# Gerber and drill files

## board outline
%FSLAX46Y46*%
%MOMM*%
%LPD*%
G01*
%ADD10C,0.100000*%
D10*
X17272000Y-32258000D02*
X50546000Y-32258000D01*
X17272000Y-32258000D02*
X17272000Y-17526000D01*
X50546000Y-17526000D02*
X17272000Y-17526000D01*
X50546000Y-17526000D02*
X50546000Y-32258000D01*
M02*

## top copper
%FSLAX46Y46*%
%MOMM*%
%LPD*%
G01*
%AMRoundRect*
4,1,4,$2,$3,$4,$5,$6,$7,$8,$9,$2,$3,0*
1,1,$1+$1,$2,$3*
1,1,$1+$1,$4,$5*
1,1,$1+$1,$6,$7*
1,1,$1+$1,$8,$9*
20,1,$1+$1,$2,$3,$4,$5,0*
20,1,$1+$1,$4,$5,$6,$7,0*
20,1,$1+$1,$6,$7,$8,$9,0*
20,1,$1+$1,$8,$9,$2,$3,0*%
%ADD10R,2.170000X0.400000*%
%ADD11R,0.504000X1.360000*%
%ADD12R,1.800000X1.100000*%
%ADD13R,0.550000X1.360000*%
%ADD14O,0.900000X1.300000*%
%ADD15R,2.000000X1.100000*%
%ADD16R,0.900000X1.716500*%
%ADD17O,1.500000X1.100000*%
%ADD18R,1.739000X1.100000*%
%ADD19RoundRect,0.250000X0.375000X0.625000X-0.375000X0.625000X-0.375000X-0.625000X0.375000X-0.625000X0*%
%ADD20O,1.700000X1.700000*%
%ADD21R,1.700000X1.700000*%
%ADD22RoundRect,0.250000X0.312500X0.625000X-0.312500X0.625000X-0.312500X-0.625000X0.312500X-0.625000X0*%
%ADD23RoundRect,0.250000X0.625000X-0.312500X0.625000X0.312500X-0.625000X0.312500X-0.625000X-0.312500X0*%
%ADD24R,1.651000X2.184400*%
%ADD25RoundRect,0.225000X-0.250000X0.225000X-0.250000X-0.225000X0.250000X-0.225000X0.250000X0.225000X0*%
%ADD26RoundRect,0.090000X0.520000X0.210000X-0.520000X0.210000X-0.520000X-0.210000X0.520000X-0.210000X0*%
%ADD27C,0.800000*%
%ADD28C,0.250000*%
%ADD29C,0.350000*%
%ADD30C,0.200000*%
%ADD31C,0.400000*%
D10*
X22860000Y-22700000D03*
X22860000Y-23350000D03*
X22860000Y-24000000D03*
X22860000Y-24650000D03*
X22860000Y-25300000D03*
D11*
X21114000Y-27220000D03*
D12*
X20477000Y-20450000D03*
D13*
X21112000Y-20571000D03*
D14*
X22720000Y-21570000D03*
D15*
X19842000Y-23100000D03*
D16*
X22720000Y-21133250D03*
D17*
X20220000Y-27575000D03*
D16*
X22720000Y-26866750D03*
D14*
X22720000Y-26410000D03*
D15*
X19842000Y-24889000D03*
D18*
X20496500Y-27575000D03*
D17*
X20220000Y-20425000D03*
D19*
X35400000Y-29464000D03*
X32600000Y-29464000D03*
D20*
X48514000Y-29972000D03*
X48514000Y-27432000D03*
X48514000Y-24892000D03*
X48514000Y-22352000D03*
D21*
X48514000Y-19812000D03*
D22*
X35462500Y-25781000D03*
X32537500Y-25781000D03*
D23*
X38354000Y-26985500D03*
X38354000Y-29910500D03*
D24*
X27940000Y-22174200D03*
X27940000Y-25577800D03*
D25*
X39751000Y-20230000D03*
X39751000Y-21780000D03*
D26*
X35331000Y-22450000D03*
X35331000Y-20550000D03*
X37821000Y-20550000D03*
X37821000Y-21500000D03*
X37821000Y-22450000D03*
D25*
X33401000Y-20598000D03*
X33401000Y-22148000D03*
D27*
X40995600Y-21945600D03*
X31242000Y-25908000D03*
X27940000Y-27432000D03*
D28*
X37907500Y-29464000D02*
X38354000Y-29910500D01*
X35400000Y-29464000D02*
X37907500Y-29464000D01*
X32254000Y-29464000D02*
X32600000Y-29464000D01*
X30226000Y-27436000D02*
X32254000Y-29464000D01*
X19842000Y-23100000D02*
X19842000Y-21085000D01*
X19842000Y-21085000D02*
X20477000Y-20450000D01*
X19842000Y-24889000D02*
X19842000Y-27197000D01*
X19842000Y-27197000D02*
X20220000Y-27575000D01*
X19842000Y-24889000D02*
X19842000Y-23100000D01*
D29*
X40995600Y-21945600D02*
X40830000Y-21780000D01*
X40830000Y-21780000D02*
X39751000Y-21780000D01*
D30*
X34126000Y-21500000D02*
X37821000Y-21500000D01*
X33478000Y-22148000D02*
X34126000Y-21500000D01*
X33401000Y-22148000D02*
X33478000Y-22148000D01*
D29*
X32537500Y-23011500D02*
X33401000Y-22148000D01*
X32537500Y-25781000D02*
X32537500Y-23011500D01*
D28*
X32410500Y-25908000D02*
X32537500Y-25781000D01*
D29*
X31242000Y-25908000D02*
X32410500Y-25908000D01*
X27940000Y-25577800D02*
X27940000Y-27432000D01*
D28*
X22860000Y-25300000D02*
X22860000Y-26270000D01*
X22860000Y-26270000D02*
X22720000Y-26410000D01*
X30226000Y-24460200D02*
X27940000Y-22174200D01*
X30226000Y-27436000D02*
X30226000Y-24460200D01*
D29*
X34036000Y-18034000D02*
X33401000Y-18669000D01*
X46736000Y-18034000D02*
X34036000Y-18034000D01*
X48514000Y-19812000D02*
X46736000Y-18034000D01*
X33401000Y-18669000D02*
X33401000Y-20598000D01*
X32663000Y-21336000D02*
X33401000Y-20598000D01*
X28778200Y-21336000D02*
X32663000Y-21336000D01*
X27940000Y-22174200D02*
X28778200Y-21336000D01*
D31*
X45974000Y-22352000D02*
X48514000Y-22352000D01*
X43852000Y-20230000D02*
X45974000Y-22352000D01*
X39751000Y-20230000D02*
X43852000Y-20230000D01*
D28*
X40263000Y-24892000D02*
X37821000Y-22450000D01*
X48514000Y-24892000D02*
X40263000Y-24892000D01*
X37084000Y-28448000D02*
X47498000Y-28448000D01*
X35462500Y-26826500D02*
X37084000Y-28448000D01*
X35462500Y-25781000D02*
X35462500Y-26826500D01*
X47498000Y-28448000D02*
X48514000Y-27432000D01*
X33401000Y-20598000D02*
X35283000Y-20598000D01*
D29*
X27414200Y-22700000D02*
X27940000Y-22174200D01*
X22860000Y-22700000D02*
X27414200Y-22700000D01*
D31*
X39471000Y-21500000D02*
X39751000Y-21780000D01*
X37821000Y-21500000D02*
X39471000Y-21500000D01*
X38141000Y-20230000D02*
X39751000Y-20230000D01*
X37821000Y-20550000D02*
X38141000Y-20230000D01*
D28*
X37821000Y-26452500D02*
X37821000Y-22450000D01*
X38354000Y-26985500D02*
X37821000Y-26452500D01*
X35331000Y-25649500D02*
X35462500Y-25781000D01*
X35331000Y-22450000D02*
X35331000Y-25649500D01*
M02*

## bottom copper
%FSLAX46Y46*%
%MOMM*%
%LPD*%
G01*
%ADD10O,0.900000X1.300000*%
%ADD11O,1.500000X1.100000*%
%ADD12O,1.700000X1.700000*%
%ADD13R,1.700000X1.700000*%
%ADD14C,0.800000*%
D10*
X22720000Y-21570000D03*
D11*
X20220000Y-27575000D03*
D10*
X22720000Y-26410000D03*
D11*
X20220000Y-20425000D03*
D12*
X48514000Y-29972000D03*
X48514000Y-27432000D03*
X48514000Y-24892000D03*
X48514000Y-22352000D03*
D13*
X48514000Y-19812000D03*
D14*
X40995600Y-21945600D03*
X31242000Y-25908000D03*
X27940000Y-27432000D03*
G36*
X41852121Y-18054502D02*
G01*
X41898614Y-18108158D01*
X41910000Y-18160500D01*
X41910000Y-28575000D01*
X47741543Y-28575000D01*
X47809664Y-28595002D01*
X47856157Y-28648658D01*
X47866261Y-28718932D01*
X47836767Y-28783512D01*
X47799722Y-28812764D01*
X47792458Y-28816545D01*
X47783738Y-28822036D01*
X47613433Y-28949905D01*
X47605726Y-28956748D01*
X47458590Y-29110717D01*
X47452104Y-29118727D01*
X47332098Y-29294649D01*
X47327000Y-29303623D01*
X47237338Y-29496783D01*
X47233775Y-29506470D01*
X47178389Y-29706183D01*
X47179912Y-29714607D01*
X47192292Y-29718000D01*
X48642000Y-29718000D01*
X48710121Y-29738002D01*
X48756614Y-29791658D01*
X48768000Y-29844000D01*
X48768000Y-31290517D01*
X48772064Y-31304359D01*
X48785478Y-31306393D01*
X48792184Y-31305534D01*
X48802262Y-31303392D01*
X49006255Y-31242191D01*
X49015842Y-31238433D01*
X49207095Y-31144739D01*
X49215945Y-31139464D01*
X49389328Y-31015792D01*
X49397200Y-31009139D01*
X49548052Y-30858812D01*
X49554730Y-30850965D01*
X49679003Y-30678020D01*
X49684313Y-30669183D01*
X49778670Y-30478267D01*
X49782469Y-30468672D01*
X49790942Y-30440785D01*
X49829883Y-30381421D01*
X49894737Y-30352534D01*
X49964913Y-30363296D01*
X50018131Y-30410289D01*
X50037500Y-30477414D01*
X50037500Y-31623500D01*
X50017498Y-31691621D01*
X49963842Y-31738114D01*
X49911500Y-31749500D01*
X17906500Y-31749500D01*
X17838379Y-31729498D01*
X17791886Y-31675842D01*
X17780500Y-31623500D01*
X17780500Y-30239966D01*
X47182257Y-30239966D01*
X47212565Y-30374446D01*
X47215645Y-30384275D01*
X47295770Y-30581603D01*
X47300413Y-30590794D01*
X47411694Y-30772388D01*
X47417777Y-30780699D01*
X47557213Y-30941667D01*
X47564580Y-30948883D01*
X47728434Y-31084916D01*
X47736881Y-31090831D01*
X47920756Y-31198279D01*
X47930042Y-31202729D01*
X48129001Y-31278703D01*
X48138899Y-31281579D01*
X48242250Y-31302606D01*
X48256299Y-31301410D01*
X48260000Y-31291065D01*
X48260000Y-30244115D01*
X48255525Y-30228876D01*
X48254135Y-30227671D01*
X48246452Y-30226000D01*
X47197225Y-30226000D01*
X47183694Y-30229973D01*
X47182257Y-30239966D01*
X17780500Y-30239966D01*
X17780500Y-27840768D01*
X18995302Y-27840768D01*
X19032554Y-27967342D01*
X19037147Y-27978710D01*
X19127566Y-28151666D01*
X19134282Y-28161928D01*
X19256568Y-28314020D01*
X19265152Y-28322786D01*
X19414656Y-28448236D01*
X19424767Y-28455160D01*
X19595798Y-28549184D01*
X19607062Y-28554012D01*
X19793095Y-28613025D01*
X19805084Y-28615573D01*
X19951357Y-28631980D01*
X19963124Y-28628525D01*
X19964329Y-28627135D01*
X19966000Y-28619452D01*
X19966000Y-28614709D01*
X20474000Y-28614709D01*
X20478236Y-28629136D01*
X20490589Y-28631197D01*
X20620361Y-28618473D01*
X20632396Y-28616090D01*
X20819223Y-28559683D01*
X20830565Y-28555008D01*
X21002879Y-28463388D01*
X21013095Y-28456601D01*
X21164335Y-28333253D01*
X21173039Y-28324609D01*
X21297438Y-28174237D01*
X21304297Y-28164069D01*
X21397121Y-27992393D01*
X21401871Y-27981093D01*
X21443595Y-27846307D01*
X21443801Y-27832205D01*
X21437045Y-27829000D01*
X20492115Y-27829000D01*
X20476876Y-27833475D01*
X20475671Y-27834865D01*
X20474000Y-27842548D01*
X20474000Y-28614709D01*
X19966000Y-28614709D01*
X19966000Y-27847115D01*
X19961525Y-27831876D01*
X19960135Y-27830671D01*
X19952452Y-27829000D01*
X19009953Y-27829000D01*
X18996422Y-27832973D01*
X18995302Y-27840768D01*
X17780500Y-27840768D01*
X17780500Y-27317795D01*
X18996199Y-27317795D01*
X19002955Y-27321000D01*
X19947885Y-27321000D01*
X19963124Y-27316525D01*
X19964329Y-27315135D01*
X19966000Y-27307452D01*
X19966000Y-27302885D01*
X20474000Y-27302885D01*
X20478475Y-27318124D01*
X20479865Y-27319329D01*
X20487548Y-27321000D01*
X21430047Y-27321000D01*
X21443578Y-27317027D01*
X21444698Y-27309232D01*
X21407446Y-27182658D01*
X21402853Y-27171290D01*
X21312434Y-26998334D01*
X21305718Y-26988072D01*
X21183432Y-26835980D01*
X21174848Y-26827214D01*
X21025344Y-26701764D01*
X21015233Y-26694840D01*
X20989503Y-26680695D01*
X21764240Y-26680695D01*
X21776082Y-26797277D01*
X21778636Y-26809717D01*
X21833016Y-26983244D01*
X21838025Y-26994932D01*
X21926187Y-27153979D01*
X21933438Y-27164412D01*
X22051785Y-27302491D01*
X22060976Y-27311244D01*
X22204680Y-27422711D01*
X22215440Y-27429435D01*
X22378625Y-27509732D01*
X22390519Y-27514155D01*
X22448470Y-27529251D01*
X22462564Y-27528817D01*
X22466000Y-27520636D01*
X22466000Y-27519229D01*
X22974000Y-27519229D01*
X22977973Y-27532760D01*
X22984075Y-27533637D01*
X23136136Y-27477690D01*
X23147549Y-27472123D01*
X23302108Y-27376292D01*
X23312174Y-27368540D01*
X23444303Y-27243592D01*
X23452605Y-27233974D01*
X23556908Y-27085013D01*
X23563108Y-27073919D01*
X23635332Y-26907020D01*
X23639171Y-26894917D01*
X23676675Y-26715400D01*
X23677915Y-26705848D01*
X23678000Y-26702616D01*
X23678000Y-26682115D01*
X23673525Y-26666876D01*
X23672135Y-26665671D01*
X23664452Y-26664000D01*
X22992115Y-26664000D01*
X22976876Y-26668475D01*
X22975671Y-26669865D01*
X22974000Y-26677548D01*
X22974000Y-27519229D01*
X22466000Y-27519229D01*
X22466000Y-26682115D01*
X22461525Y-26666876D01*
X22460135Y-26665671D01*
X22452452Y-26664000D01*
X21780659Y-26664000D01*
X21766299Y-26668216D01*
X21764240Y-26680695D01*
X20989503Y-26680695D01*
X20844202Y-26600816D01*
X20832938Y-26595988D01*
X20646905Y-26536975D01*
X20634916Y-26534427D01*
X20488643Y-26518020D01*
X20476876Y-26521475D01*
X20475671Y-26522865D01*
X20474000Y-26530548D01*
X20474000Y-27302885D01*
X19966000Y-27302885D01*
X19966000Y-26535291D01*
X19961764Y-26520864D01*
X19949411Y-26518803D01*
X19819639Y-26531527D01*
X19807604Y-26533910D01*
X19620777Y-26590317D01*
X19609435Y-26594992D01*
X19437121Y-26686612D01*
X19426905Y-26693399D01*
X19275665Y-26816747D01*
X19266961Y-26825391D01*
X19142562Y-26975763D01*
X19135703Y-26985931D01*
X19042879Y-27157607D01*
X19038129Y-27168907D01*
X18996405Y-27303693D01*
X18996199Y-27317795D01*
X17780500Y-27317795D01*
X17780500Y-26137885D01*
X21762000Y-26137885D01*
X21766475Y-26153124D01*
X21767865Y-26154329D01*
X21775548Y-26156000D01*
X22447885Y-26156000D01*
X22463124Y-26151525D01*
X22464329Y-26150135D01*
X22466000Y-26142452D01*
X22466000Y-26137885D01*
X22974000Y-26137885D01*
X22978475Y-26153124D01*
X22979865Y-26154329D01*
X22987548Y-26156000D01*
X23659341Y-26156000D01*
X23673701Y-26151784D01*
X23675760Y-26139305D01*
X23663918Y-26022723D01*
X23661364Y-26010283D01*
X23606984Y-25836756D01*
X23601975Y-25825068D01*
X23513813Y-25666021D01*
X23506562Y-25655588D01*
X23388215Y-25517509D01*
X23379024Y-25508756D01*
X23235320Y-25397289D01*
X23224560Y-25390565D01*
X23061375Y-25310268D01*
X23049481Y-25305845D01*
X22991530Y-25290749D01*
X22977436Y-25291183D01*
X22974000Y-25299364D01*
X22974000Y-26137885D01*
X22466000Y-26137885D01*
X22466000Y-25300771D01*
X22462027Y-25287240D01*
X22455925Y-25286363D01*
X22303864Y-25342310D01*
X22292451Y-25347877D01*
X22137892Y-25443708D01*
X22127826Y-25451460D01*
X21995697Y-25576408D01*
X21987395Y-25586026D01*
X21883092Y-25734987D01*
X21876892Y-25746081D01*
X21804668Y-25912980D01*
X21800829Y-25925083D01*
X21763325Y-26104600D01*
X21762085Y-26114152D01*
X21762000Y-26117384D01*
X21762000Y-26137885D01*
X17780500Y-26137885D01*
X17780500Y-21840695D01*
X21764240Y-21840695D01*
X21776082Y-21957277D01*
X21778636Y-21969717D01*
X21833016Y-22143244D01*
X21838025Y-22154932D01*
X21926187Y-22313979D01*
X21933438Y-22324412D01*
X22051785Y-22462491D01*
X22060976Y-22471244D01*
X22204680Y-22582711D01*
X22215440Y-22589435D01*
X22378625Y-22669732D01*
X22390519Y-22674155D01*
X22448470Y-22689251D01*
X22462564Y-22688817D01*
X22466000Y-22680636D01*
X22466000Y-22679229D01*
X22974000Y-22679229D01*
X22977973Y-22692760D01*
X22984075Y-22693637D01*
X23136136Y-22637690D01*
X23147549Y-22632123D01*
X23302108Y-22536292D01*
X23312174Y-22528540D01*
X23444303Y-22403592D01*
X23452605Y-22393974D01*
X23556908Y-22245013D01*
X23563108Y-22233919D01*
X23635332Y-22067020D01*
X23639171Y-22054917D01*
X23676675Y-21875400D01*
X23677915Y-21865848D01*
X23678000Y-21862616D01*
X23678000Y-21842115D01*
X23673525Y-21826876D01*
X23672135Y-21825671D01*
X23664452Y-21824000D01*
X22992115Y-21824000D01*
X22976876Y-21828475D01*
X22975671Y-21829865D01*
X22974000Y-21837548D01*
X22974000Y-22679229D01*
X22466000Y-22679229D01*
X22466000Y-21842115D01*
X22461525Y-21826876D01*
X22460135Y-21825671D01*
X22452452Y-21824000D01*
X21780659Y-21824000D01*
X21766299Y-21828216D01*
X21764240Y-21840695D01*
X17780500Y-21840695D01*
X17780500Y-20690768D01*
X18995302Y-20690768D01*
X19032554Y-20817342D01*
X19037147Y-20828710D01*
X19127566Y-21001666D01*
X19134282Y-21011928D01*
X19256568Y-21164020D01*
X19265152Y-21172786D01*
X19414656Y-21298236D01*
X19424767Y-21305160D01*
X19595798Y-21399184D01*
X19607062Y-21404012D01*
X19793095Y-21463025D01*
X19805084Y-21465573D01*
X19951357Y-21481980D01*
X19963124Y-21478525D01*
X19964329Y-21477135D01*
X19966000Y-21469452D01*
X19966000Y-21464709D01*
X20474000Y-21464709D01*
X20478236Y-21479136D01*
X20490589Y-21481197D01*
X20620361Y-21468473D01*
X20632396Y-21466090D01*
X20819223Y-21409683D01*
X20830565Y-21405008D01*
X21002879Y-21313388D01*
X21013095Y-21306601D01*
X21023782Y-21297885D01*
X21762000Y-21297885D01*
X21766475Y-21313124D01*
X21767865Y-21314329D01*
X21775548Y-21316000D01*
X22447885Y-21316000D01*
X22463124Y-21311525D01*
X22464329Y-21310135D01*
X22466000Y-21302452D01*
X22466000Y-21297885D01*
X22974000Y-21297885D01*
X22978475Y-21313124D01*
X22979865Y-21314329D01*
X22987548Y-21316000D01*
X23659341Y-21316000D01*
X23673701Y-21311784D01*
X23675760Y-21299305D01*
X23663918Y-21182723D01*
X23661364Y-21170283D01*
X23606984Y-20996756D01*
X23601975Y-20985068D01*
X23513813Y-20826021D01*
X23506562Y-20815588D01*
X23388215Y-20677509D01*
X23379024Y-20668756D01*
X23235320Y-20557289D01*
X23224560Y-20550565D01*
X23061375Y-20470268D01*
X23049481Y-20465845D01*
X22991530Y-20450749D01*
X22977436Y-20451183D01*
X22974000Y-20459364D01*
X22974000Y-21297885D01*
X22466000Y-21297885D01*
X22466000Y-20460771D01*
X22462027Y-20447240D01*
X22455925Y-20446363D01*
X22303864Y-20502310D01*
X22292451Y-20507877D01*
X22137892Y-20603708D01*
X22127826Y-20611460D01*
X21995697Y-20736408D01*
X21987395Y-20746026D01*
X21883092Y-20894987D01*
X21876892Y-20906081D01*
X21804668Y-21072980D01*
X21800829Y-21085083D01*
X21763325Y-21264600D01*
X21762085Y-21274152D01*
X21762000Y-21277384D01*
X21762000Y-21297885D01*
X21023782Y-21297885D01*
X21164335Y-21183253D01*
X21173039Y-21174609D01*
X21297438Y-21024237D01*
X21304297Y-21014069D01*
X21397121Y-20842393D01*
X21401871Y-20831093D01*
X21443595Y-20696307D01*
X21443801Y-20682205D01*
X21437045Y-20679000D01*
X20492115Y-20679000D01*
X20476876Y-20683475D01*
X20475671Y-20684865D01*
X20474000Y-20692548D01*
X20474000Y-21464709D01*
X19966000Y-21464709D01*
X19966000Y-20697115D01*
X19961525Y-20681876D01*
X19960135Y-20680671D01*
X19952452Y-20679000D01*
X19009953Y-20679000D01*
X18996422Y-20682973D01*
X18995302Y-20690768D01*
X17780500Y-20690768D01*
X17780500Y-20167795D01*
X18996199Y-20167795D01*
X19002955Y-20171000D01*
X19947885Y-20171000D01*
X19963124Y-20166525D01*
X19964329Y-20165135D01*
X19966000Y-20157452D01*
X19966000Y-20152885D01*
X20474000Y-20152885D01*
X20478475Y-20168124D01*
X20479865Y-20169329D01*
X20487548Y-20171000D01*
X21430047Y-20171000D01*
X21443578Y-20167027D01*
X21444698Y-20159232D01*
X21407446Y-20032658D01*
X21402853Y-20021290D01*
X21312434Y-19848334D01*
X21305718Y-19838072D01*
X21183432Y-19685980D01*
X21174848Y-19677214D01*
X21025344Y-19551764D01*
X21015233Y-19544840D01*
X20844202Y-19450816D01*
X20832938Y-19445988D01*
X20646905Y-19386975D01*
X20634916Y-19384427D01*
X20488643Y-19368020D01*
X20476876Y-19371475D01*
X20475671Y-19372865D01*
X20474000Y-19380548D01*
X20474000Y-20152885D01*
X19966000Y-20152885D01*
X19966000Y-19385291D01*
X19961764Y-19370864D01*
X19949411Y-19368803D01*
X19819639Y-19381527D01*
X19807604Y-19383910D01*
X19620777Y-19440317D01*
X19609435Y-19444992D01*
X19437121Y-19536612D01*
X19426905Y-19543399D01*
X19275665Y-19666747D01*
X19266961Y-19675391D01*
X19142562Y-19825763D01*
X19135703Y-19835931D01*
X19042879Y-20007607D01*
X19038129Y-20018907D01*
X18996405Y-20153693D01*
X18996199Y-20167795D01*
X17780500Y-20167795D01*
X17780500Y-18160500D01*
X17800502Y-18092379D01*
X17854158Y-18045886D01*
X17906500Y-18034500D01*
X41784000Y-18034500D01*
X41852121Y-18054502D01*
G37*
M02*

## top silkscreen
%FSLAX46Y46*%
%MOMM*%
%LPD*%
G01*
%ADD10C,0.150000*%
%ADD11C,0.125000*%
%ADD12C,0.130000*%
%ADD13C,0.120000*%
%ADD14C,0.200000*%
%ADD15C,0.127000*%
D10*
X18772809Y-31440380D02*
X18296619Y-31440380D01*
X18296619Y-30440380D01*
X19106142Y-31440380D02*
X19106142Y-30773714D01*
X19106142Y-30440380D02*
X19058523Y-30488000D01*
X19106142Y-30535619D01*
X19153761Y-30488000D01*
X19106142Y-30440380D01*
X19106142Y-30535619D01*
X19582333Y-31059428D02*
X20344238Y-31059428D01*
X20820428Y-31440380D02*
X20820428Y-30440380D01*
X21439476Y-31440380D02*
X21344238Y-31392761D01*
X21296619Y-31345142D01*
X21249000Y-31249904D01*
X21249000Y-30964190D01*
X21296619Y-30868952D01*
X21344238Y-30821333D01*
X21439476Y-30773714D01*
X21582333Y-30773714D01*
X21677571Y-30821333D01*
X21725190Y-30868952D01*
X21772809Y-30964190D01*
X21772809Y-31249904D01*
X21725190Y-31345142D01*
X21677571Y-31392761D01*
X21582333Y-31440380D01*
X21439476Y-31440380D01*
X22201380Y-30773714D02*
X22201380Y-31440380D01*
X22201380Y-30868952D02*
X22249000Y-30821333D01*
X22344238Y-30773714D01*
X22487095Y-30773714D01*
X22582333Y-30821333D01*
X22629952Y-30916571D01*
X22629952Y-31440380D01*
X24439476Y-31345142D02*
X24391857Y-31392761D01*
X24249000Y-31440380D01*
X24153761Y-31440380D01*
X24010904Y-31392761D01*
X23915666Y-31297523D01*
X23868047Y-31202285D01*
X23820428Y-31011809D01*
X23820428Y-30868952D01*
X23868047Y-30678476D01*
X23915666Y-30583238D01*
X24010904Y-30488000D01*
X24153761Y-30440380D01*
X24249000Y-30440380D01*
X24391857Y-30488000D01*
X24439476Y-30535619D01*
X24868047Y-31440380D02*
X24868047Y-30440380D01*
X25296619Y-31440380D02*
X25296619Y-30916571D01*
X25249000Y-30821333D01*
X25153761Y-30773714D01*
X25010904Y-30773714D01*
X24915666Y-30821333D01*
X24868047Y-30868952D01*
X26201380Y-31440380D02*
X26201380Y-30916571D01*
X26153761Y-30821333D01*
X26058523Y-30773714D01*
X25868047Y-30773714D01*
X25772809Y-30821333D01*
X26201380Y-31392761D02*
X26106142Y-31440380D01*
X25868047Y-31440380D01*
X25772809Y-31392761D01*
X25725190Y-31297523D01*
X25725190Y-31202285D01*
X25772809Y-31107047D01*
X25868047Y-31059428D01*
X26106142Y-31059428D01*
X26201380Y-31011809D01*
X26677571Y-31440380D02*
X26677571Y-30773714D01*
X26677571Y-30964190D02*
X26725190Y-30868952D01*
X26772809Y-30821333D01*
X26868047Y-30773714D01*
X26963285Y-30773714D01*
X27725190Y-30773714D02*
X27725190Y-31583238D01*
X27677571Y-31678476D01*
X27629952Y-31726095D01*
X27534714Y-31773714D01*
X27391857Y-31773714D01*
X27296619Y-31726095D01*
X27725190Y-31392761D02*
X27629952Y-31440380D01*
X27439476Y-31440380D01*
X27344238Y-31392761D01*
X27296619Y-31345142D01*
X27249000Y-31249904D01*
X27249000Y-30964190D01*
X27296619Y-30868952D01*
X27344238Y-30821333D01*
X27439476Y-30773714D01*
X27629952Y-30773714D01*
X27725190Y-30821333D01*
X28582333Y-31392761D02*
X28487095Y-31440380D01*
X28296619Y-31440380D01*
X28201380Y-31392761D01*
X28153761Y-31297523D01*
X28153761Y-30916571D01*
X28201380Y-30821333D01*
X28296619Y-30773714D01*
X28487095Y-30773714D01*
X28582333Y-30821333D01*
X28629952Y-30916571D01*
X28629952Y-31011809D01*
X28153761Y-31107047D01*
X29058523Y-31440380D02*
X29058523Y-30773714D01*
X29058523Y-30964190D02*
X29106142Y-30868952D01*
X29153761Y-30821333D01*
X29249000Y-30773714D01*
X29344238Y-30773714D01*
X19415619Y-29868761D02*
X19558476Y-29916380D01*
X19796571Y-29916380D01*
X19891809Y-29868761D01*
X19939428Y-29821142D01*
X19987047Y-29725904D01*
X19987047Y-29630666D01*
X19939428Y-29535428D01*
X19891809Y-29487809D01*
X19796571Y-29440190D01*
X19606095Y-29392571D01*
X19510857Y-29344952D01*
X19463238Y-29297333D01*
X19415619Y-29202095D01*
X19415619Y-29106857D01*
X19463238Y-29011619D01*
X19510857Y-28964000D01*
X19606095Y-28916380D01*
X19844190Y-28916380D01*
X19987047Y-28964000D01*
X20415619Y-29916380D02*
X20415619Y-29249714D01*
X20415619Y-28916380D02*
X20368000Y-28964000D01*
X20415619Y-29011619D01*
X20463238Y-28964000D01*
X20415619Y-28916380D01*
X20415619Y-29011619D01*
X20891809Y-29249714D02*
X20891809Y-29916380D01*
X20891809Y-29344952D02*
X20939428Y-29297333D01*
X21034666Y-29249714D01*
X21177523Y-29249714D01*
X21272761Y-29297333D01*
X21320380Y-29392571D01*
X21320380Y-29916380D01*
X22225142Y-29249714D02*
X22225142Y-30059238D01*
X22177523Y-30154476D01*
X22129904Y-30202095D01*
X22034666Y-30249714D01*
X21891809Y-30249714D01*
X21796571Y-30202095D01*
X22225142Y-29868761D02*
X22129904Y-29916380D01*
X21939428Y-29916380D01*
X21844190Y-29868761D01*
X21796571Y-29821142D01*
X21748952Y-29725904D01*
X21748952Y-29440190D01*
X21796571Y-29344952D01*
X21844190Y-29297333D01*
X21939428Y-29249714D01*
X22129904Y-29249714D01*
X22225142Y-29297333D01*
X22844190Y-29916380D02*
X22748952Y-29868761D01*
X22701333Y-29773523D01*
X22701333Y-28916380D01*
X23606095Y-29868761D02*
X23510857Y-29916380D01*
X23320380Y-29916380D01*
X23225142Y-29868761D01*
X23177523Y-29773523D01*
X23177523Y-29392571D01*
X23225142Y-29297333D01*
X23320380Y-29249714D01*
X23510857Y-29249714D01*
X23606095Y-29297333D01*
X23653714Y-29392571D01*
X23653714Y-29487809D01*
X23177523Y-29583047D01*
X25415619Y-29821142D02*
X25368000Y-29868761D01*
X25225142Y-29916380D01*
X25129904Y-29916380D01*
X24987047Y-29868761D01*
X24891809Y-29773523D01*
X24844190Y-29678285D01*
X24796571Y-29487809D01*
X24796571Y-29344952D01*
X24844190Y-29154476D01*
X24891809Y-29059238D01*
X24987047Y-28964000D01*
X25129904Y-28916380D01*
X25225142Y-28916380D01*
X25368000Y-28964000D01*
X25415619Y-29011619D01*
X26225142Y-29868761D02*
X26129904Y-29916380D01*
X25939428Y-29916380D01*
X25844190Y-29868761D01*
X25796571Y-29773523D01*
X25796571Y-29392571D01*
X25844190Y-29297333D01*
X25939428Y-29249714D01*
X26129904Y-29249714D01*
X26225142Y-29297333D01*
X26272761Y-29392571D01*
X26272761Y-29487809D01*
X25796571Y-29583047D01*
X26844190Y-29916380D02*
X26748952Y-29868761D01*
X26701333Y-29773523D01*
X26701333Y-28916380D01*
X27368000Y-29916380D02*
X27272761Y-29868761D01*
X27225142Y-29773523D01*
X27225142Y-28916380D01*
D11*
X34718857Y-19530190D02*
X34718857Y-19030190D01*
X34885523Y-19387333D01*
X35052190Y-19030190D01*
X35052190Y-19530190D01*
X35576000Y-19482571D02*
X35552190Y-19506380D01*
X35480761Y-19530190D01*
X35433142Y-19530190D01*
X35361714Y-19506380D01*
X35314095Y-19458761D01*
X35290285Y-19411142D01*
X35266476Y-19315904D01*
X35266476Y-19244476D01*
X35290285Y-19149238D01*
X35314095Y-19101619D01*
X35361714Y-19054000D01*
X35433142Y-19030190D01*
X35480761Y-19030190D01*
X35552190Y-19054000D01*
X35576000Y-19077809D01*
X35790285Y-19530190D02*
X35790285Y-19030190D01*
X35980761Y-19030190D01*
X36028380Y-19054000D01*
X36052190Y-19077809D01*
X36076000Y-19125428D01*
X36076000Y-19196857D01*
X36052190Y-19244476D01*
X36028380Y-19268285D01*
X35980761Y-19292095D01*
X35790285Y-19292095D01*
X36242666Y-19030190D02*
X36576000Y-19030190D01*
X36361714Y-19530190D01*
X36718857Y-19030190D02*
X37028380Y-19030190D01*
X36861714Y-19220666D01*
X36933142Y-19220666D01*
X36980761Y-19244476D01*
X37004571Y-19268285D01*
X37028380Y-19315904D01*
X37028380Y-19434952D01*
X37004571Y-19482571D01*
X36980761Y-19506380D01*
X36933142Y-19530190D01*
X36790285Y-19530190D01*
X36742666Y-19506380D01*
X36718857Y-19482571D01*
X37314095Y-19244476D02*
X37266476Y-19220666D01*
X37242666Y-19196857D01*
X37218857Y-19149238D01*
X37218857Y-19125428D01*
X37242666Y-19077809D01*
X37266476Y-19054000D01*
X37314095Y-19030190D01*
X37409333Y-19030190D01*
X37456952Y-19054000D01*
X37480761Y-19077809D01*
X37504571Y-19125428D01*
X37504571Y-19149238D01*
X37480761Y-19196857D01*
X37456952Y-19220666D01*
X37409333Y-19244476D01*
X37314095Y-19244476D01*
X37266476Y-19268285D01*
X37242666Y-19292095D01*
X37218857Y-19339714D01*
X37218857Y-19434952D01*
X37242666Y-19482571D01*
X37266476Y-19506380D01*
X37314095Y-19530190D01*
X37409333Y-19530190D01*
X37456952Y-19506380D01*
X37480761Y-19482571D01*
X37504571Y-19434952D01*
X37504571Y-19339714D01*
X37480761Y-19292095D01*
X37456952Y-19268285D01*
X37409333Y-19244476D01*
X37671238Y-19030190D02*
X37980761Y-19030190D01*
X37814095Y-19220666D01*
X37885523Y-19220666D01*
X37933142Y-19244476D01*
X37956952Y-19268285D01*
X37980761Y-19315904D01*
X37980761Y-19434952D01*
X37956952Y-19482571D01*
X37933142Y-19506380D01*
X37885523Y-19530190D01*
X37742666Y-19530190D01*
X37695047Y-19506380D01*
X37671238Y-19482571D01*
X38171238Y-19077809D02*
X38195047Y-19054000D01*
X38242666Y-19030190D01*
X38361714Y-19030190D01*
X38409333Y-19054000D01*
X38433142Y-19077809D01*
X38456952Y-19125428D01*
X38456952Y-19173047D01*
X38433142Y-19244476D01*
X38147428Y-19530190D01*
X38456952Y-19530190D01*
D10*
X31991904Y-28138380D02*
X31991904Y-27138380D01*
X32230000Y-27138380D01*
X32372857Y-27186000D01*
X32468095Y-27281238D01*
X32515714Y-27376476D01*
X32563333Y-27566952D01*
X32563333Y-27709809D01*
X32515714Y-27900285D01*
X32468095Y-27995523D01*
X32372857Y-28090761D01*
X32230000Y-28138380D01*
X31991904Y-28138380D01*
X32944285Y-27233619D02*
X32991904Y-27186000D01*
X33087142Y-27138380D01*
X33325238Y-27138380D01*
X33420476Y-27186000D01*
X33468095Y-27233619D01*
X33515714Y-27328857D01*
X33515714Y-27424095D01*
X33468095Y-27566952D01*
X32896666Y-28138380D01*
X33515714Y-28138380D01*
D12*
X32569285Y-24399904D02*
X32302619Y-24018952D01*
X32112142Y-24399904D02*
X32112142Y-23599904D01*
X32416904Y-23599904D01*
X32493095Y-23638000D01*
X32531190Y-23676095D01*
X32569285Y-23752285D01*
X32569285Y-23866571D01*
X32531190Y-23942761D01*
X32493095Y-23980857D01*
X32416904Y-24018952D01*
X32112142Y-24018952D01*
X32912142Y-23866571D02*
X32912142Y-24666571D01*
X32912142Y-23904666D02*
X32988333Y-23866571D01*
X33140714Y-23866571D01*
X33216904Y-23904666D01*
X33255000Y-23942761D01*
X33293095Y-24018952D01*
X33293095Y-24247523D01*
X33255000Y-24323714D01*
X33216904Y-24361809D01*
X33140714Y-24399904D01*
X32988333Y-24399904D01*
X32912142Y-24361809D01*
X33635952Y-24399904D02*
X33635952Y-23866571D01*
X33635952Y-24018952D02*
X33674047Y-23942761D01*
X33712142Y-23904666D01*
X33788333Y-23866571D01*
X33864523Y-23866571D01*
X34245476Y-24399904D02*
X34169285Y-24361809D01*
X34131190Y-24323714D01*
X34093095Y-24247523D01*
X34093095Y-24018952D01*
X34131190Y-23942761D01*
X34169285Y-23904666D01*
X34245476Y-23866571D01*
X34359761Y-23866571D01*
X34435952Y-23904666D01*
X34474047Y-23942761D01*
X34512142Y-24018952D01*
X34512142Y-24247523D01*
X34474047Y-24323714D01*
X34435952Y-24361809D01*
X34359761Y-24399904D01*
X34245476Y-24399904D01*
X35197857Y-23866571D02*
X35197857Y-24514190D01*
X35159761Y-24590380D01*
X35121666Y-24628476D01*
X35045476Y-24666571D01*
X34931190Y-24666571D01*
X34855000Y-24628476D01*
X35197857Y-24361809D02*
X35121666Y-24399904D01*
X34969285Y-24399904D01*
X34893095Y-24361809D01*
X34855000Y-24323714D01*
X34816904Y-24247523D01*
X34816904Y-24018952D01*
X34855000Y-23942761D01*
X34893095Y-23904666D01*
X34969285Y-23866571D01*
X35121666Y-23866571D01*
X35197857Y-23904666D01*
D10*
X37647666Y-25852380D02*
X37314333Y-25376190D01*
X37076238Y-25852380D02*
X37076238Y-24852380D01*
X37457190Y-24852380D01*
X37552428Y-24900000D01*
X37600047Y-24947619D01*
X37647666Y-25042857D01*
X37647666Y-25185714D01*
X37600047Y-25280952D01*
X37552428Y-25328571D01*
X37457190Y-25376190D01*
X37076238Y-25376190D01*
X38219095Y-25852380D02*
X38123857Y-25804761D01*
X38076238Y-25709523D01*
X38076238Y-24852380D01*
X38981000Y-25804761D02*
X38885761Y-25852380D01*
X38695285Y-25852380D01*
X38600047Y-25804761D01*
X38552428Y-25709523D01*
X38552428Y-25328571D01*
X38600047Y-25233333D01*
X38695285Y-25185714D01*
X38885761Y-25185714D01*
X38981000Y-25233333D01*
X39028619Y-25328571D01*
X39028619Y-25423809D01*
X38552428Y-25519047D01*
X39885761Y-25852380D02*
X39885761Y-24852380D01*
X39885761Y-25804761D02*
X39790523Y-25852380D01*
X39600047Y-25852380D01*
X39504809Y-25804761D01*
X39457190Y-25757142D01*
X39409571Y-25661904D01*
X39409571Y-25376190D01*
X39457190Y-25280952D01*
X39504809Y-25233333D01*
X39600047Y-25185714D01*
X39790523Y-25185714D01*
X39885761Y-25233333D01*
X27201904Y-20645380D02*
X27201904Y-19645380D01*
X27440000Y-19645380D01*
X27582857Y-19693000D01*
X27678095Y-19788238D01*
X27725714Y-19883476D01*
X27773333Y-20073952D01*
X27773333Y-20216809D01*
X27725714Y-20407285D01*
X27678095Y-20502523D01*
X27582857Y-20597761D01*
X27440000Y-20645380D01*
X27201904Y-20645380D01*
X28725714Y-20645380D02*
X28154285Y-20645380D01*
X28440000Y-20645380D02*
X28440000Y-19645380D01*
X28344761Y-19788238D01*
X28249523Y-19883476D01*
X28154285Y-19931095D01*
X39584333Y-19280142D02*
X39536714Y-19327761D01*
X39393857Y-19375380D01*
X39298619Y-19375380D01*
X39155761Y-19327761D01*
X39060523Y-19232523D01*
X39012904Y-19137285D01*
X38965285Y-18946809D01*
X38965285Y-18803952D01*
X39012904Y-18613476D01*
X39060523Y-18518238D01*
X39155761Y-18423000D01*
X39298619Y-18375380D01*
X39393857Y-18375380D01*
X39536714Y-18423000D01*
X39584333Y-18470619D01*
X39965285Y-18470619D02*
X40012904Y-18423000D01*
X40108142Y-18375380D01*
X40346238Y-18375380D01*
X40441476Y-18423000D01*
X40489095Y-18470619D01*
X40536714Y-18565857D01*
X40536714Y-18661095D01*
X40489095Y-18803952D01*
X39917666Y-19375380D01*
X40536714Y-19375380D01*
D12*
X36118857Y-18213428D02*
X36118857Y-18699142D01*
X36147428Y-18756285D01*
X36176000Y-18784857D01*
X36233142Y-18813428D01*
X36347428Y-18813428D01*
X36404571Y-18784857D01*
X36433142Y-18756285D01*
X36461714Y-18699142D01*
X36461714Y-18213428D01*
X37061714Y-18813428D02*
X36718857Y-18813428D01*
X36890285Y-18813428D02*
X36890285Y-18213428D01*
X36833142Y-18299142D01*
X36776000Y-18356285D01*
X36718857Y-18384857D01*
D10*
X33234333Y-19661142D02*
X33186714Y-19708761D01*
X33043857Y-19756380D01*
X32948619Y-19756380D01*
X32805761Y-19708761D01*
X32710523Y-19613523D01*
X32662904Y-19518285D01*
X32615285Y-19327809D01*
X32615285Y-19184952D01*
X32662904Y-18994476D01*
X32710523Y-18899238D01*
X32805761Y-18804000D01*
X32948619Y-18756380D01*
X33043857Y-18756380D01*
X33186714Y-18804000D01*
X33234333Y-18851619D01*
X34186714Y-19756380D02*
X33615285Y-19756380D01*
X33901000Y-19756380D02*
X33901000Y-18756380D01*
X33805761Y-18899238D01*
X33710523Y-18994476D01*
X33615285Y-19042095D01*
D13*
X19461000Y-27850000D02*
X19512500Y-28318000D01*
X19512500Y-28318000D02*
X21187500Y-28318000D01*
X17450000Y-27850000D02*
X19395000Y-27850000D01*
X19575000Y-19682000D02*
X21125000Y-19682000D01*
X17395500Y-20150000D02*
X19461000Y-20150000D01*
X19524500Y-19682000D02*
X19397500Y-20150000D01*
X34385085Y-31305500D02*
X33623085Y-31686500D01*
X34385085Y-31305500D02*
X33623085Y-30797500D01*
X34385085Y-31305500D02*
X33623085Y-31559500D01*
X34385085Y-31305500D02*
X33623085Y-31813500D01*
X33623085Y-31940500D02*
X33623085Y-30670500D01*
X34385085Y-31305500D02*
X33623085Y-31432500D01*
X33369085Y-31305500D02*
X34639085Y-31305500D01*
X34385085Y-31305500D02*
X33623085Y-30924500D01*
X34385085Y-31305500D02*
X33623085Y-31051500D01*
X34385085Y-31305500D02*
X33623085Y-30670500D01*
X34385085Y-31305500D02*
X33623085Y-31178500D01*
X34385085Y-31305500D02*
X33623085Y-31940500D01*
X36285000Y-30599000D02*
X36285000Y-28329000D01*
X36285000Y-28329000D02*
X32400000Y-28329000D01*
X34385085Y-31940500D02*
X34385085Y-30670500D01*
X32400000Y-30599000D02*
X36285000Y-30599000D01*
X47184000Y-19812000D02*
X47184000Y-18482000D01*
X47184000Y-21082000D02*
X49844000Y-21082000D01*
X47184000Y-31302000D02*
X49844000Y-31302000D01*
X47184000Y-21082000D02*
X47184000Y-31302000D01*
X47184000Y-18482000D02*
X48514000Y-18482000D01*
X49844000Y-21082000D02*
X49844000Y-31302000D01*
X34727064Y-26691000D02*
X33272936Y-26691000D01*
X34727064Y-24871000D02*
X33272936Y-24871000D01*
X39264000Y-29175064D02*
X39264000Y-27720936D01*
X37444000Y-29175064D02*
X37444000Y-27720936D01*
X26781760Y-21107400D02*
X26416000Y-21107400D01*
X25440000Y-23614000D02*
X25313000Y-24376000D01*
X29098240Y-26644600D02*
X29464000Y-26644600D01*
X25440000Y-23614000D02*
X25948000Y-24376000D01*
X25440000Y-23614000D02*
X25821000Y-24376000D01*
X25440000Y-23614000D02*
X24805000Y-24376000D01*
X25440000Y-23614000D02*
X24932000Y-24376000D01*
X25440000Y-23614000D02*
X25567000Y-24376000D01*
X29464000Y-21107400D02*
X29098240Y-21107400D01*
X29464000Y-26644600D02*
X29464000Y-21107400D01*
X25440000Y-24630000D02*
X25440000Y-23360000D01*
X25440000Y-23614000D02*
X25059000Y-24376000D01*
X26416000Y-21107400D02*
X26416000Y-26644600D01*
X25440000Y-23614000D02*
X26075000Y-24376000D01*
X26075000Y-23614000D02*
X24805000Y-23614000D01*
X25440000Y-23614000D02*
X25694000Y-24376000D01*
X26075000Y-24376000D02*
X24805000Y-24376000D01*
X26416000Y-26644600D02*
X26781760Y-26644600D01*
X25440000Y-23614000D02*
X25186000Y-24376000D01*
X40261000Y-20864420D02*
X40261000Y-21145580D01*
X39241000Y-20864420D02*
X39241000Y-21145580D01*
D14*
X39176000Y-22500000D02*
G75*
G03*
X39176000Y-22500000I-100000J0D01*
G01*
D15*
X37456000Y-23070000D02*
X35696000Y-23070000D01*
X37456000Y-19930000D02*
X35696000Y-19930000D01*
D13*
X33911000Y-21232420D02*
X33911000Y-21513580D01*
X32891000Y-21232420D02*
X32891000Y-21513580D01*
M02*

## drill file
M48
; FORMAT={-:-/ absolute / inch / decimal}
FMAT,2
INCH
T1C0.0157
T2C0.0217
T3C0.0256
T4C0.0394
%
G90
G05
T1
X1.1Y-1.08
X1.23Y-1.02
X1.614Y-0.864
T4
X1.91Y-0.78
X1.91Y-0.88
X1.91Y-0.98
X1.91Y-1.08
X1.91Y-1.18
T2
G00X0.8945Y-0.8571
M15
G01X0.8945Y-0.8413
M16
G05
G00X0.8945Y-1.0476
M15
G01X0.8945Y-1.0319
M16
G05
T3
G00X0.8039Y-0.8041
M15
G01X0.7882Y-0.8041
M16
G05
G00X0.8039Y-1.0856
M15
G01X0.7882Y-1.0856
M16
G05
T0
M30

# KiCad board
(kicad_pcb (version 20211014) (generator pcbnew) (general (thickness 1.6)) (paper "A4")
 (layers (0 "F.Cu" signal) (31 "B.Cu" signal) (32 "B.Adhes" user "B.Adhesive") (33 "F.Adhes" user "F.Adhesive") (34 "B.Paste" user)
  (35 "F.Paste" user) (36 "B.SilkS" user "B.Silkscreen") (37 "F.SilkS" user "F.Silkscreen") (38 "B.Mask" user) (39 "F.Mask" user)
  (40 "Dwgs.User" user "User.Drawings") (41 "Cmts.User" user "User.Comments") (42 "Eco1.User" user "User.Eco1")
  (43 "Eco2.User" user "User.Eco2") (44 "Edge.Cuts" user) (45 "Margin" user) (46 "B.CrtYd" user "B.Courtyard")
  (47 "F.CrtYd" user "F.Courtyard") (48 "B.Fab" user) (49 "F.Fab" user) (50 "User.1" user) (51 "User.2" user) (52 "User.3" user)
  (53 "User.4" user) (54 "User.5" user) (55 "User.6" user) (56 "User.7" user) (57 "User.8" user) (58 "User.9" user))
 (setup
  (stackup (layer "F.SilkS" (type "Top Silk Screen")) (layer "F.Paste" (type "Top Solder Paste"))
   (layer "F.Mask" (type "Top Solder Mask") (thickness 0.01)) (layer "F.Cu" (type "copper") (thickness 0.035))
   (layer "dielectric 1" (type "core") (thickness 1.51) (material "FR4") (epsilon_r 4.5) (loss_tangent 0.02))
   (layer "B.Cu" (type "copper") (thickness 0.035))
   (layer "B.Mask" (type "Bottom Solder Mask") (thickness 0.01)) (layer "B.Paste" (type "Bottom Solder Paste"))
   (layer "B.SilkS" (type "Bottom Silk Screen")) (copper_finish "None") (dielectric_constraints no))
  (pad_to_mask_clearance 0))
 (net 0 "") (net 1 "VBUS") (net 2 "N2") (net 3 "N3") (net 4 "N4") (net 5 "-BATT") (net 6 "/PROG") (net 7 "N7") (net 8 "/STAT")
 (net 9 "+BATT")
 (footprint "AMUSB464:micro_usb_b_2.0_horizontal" (layer "F.Cu") (at 18.445 24 -90)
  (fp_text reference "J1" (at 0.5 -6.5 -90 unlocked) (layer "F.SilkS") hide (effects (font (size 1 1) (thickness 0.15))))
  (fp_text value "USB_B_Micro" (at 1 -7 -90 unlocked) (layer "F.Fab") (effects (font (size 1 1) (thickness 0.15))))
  (fp_line (start 4.318 -1.0675) (end 4.318 -2.7425) (layer "F.SilkS") (width 0.12))
  (fp_line (start 3.85 -1.016) (end 4.318 -1.0675) (layer "F.SilkS") (width 0.12))
  (fp_line (start -4.318 -1.0795) (end -3.85 -0.9525) (layer "F.SilkS") (width 0.12))
  (fp_line (start -4.318 -1.13) (end -4.318 -2.68) (layer "F.SilkS") (width 0.12))
  (fp_line (start -3.85 1.0495) (end -3.85 -1.016) (layer "F.SilkS") (width 0.12))
  (fp_line (start 3.85 0.995) (end 3.85 -0.95) (layer "F.SilkS") (width 0.12))
  (pad "1" smd rect (at -1.3 -4.415) (size 2.17 0.4) (layers "F.Cu" "F.Paste" "F.Mask") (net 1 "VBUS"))
  (pad "2" smd rect (at -0.65 -4.415) (size 2.17 0.4) (layers "F.Cu" "F.Paste" "F.Mask") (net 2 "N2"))
  (pad "3" smd rect (at 0 -4.415) (size 2.17 0.4) (layers "F.Cu" "F.Paste" "F.Mask") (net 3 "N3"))
  (pad "4" smd rect (at 0.65 -4.415) (size 2.17 0.4) (layers "F.Cu" "F.Paste" "F.Mask") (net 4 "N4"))
  (pad "5" smd rect (at 1.3 -4.415) (size 2.17 0.4) (layers "F.Cu" "F.Paste" "F.Mask") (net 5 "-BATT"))
  (pad "6" thru_hole oval (at -2.43 -4.275 90) (size 1.3 0.9) (drill oval 0.95 0.55) (layers *.Cu *.Mask) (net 5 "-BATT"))
  (pad "6" smd rect (at -2.86675 -4.275 270) (size 1.7165 0.9) (layers "F.Cu" "F.Paste" "F.Mask") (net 5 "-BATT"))
  (pad "6" thru_hole oval (at -3.575 -1.775 180) (size 1.5 1.1) (drill oval 1.05 0.65) (layers *.Cu *.Mask) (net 5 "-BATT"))
  (pad "6" smd rect (at 2.86675 -4.275 270) (size 1.7165 0.9) (layers "F.Cu" "F.Paste" "F.Mask") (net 5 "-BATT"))
  (pad "6" thru_hole oval (at 2.41 -4.275 90) (size 1.3 0.9) (drill oval 0.95 0.55) (layers *.Cu *.Mask) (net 5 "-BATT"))
  (pad "6" smd rect (at 3.22 -2.669 270) (size 1.36 0.504) (layers "F.Cu" "F.Paste" "F.Mask") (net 5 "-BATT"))
  (pad "6" smd rect (at -0.9 -1.397 180) (size 2 1.1) (layers "F.Cu" "F.Paste" "F.Mask") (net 5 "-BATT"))
  (pad "6" smd rect (at 0.889 -1.397 180) (size 2 1.1) (layers "F.Cu" "F.Paste" "F.Mask") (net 5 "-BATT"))
  (pad "6" smd rect (at -3.55 -2.032) (size 1.8 1.1) (layers "F.Cu" "F.Paste" "F.Mask") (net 5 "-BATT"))
  (pad "6" smd rect (at -3.429 -2.667 270) (size 1.36 0.55) (layers "F.Cu" "F.Paste" "F.Mask") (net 5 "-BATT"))
  (pad "6" thru_hole oval (at 3.575 -1.775 180) (size 1.5 1.1) (drill oval 1.05 0.65) (layers *.Cu *.Mask) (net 5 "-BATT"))
  (pad "6" smd rect (at 3.575 -2.0515 180) (size 1.739 1.1) (layers "F.Cu" "F.Paste" "F.Mask") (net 5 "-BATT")))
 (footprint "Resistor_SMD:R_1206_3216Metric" (layer "F.Cu") (at 34 25.781 180)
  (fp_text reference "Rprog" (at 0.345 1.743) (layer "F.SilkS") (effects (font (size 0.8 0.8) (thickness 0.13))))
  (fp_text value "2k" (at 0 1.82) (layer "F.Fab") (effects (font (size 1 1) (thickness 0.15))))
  (fp_line (start -0.727064 -0.91) (end 0.727064 -0.91) (layer "F.SilkS") (width 0.12))
  (fp_line (start -0.727064 0.91) (end 0.727064 0.91) (layer "F.SilkS") (width 0.12))
  (pad "1" smd roundrect (at -1.4625 0 180) (size 1.125 1.75) (layers "F.Cu" "F.Paste" "F.Mask") (roundrect_rratio 0.2222222222)
   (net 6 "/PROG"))
  (pad "2" smd roundrect (at 1.4625 0 180) (size 1.125 1.75) (layers "F.Cu" "F.Paste" "F.Mask") (roundrect_rratio 0.2222222222)
   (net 5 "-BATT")))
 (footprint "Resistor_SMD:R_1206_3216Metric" (layer "F.Cu") (at 38.354 28.448 90)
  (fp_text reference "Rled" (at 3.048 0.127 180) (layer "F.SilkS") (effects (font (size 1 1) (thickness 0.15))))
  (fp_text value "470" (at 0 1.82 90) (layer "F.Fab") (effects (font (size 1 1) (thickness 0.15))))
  (fp_line (start -0.727064 -0.91) (end 0.727064 -0.91) (layer "F.SilkS") (width 0.12))
  (fp_line (start -0.727064 0.91) (end 0.727064 0.91) (layer "F.SilkS") (width 0.12))
  (pad "1" smd roundrect (at -1.4625 0 90) (size 1.125 1.75) (layers "F.Cu" "F.Paste" "F.Mask") (roundrect_rratio 0.2222222222) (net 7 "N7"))
  (pad "2" smd roundrect (at 1.4625 0 90) (size 1.125 1.75) (layers "F.Cu" "F.Paste" "F.Mask") (roundrect_rratio 0.2222222222)
   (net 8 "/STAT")))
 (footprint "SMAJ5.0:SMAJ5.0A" (layer "F.Cu") (at 27.94 23.876 -90)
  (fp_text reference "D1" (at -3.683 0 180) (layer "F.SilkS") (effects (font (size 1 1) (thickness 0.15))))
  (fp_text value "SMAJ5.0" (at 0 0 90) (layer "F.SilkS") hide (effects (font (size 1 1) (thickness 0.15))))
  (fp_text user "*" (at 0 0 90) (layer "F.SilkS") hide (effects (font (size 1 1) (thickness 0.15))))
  (fp_line (start -2.7686 1.15824) (end -2.7686 1.524) (layer "F.SilkS") (width 0.12))
  (fp_line (start -0.262 2.5) (end 0.5 2.627) (layer "F.SilkS") (width 0.12))
  (fp_line (start 2.7686 -1.15824) (end 2.7686 -1.524) (layer "F.SilkS") (width 0.12))
  (fp_line (start -0.262 2.5) (end 0.5 1.992) (layer "F.SilkS") (width 0.12))
  (fp_line (start -0.262 2.5) (end 0.5 2.119) (layer "F.SilkS") (width 0.12))
  (fp_line (start -0.262 2.5) (end 0.5 3.135) (layer "F.SilkS") (width 0.12))
  (fp_line (start -0.262 2.5) (end 0.5 3.008) (layer "F.SilkS") (width 0.12))
  (fp_line (start -0.262 2.5) (end 0.5 2.373) (layer "F.SilkS") (width 0.12))
  (fp_line (start -2.7686 -1.524) (end -2.7686 -1.15824) (layer "F.SilkS") (width 0.12))
  (fp_line (start 2.7686 -1.524) (end -2.7686 -1.524) (layer "F.SilkS") (width 0.12))
  (fp_line (start 0.754 2.5) (end -0.516 2.5) (layer "F.SilkS") (width 0.12))
  (fp_line (start -0.262 2.5) (end 0.5 2.881) (layer "F.SilkS") (width 0.12))
  (fp_line (start -2.7686 1.524) (end 2.7686 1.524) (layer "F.SilkS") (width 0.12))
  (fp_line (start -0.262 2.5) (end 0.5 1.865) (layer "F.SilkS") (width 0.12))
  (fp_line (start -0.262 1.865) (end -0.262 3.135) (layer "F.SilkS") (width 0.12))
  (fp_line (start -0.262 2.5) (end 0.5 2.246) (layer "F.SilkS") (width 0.12))
  (fp_line (start 0.5 1.865) (end 0.5 3.135) (layer "F.SilkS") (width 0.12))
  (fp_line (start 2.7686 1.524) (end 2.7686 1.15824) (layer "F.SilkS") (width 0.12))
  (fp_line (start -0.262 2.5) (end 0.5 2.754) (layer "F.SilkS") (width 0.12))
  (pad "1" smd rect (at -1.7018 0) (size 1.651 2.1844) (layers "F.Cu" "F.Paste" "F.Mask") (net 1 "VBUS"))
  (pad "2" smd rect (at 1.7018 0) (size 1.651 2.1844) (layers "F.Cu" "F.Paste" "F.Mask") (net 5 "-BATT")))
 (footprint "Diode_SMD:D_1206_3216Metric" (layer "F.Cu") (at 34 29.464 180)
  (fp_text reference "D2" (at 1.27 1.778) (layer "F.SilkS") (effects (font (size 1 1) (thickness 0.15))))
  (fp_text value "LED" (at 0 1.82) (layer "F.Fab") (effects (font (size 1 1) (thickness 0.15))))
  (fp_line (start -0.385085 -1.8415) (end 0.376915 -2.2225) (layer "F.SilkS") (width 0.12))
  (fp_line (start -0.385085 -1.8415) (end 0.376915 -1.3335) (layer "F.SilkS") (width 0.12))
  (fp_line (start -0.385085 -1.8415) (end 0.376915 -2.0955) (layer "F.SilkS") (width 0.12))
  (fp_line (start -0.385085 -1.8415) (end 0.376915 -2.3495) (layer "F.SilkS") (width 0.12))
  (fp_line (start 0.376915 -2.4765) (end 0.376915 -1.2065) (layer "F.SilkS") (width 0.12))
  (fp_line (start -0.385085 -1.8415) (end 0.376915 -1.9685) (layer "F.SilkS") (width 0.12))
  (fp_line (start 0.630915 -1.8415) (end -0.639085 -1.8415) (layer "F.SilkS") (width 0.12))
  (fp_line (start -0.385085 -1.8415) (end 0.376915 -1.4605) (layer "F.SilkS") (width 0.12))
  (fp_line (start -0.385085 -1.8415) (end 0.376915 -1.5875) (layer "F.SilkS") (width 0.12))
  (fp_line (start -0.385085 -1.8415) (end 0.376915 -1.2065) (layer "F.SilkS") (width 0.12))
  (fp_line (start -0.385085 -1.8415) (end 0.376915 -1.7145) (layer "F.SilkS") (width 0.12))
  (fp_line (start -0.385085 -1.8415) (end 0.376915 -2.4765) (layer "F.SilkS") (width 0.12))
  (fp_line (start -2.285 -1.135) (end -2.285 1.135) (layer "F.SilkS") (width 0.12))
  (fp_line (start -2.285 1.135) (end 1.6 1.135) (layer "F.SilkS") (width 0.12))
  (fp_line (start -0.385085 -2.4765) (end -0.385085 -1.2065) (layer "F.SilkS") (width 0.12))
  (fp_line (start 1.6 -1.135) (end -2.285 -1.135) (layer "F.SilkS") (width 0.12))
  (pad "1" smd roundrect (at -1.4 0 180) (size 1.25 1.75) (layers "F.Cu" "F.Paste" "F.Mask") (roundrect_rratio 0.2) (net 7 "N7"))
  (pad "2" smd roundrect (at 1.4 0 180) (size 1.25 1.75) (layers "F.Cu" "F.Paste" "F.Mask") (roundrect_rratio 0.2) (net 1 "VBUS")))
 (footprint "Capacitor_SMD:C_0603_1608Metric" (layer "F.Cu") (at 39.751 21.005 -90)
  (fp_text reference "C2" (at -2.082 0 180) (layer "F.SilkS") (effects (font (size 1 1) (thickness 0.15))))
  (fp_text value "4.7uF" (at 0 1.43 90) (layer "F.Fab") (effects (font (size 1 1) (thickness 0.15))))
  (fp_line (start -0.14058 -0.51) (end 0.14058 -0.51) (layer "F.SilkS") (width 0.12))
  (fp_line (start -0.14058 0.51) (end 0.14058 0.51) (layer "F.SilkS") (width 0.12))
  (pad "1" smd roundrect (at -0.775 0 270) (size 0.9 0.95) (layers "F.Cu" "F.Paste" "F.Mask") (roundrect_rratio 0.25) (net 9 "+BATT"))
  (pad "2" smd roundrect (at 0.775 0 270) (size 0.9 0.95) (layers "F.Cu" "F.Paste" "F.Mask") (roundrect_rratio 0.25) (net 5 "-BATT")))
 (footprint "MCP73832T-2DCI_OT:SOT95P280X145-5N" (layer "F.Cu") (at 36.576 21.5 180)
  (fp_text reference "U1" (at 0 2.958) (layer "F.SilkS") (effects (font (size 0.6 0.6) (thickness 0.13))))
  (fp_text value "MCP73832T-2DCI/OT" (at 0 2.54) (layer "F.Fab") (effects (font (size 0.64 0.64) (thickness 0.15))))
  (fp_line (start -0.88 1.57) (end 0.88 1.57) (layer "F.SilkS") (width 0.127))
  (fp_line (start -0.88 -1.57) (end 0.88 -1.57) (layer "F.SilkS") (width 0.127))
  (fp_circle (center -2.5 -1) (end -2.4 -1) (layer "F.SilkS") (width 0.2) (fill none))
  (pad "1" smd roundrect locked (at -1.245 -0.95 180) (size 1.22 0.6) (layers "F.Cu" "F.Paste" "F.Mask") (roundrect_rratio 0.15)
   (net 8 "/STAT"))
  (pad "2" smd roundrect locked (at -1.245 0 180) (size 1.22 0.6) (layers "F.Cu" "F.Paste" "F.Mask") (roundrect_rratio 0.15) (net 5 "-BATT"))
  (pad "3" smd roundrect locked (at -1.245 0.95 180) (size 1.22 0.6) (layers "F.Cu" "F.Paste" "F.Mask") (roundrect_rratio 0.15)
   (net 9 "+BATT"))
  (pad "4" smd roundrect locked (at 1.245 0.95 180) (size 1.22 0.6) (layers "F.Cu" "F.Paste" "F.Mask") (roundrect_rratio 0.15)
   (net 1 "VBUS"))
  (pad "5" smd roundrect locked (at 1.245 -0.95 180) (size 1.22 0.6) (layers "F.Cu" "F.Paste" "F.Mask") (roundrect_rratio 0.15)
   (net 6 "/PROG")))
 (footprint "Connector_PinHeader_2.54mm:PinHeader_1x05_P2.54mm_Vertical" (layer "F.Cu") (at 48.514 19.812)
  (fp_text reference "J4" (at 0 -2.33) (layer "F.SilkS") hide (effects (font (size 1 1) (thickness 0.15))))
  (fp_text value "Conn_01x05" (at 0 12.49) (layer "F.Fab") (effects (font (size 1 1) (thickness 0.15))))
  (fp_line (start -1.33 0) (end -1.33 -1.33) (layer "F.SilkS") (width 0.12))
  (fp_line (start -1.33 1.27) (end -1.33 11.49) (layer "F.SilkS") (width 0.12))
  (fp_line (start -1.33 1.27) (end 1.33 1.27) (layer "F.SilkS") (width 0.12))
  (fp_line (start -1.33 -1.33) (end 0 -1.33) (layer "F.SilkS") (width 0.12))
  (fp_line (start -1.33 11.49) (end 1.33 11.49) (layer "F.SilkS") (width 0.12))
  (fp_line (start 1.33 1.27) (end 1.33 11.49) (layer "F.SilkS") (width 0.12))
  (pad "1" thru_hole rect (at 0 0) (size 1.7 1.7) (drill 1) (layers *.Cu *.Mask) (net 1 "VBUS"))
  (pad "2" thru_hole oval (at 0 2.54) (size 1.7 1.7) (drill 1) (layers *.Cu *.Mask) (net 9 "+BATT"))
  (pad "3" thru_hole oval (at 0 5.08) (size 1.7 1.7) (drill 1) (layers *.Cu *.Mask) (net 8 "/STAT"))
  (pad "4" thru_hole oval (at 0 7.62) (size 1.7 1.7) (drill 1) (layers *.Cu *.Mask) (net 6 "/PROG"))
  (pad "5" thru_hole oval (at 0 10.16) (size 1.7 1.7) (drill 1) (layers *.Cu *.Mask) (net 5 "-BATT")))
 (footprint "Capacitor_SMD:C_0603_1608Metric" (layer "F.Cu") (at 33.401 21.373 -90)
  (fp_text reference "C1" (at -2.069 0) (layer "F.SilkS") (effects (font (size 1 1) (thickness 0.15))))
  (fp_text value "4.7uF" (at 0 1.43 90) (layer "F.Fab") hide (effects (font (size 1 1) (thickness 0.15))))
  (fp_line (start -0.14058 -0.51) (end 0.14058 -0.51) (layer "F.SilkS") (width 0.12))
  (fp_line (start -0.14058 0.51) (end 0.14058 0.51) (layer "F.SilkS") (width 0.12))
  (pad "1" smd roundrect (at -0.775 0 270) (size 0.9 0.95) (layers "F.Cu" "F.Paste" "F.Mask") (roundrect_rratio 0.25) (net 1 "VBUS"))
  (pad "2" smd roundrect (at 0.775 0 270) (size 0.9 0.95) (layers "F.Cu" "F.Paste" "F.Mask") (roundrect_rratio 0.25) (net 5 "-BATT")))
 (gr_line (start 17.272 32.258) (end 50.546 32.258) (layer "Edge.Cuts") (width 0.1))
 (gr_line (start 17.272 32.258) (end 17.272 17.526) (layer "Edge.Cuts") (width 0.1))
 (gr_line (start 50.546 17.526) (end 17.272 17.526) (layer "Edge.Cuts") (width 0.1))
 (gr_line (start 50.546 17.526) (end 50.546 32.258) (layer "Edge.Cuts") (width 0.1))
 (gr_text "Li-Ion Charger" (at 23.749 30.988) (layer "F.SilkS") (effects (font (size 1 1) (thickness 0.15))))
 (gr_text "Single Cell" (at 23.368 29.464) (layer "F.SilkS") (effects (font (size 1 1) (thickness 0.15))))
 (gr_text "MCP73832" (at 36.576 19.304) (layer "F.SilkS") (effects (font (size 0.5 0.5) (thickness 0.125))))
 (segment (start 33.478 22.148) (end 34.126 21.5) (width 0.2) (layer "F.Cu") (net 5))
 (segment (start 19.842 27.197) (end 20.22 27.575) (width 0.25) (layer "F.Cu") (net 5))
 (segment (start 40.83 21.78) (end 39.751 21.78) (width 0.35) (layer "F.Cu") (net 5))
 (segment (start 19.842 24.889) (end 19.842 27.197) (width 0.25) (layer "F.Cu") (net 5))
 (segment (start 31.242 25.908) (end 32.4105 25.908) (width 0.35) (layer "F.Cu") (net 5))
 (segment (start 40.9956 21.9456) (end 40.83 21.78) (width 0.35) (layer "F.Cu") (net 5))
 (segment (start 32.5375 23.0115) (end 33.401 22.148) (width 0.35) (layer "F.Cu") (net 5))
 (segment (start 27.94 25.5778) (end 27.94 27.432) (width 0.35) (layer "F.Cu") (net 5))
 (segment (start 19.842 24.889) (end 19.842 23.1) (width 0.25) (layer "F.Cu") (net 5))
 (segment (start 34.126 21.5) (end 37.821 21.5) (width 0.2) (layer "F.Cu") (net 5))
 (segment (start 33.401 22.148) (end 33.478 22.148) (width 0.2) (layer "F.Cu") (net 5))
 (segment (start 39.471 21.5) (end 39.751 21.78) (width 0.4) (layer "F.Cu") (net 5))
 (segment (start 37.821 21.5) (end 39.471 21.5) (width 0.4) (layer "F.Cu") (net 5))
 (segment (start 32.4105 25.908) (end 32.5375 25.781) (width 0.25) (layer "F.Cu") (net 5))
 (segment (start 32.5375 25.781) (end 32.5375 23.0115) (width 0.35) (layer "F.Cu") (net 5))
 (segment (start 22.86 25.3) (end 22.86 26.27) (width 0.25) (layer "F.Cu") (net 5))
 (segment (start 19.842 23.1) (end 19.842 21.085) (width 0.25) (layer "F.Cu") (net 5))
 (segment (start 19.842 21.085) (end 20.477 20.45) (width 0.25) (layer "F.Cu") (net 5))
 (segment (start 22.86 26.27) (end 22.72 26.41) (width 0.25) (layer "F.Cu") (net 5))
 (via (at 27.94 27.432) (size 0.8) (drill 0.4) (layers "F.Cu" "B.Cu") (free) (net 5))
 (via (at 31.242 25.908) (size 0.8) (drill 0.4) (layers "F.Cu" "B.Cu") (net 5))
 (via (at 40.9956 21.9456) (size 0.8) (drill 0.4) (layers "F.Cu" "B.Cu") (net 5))
 (segment (start 45.974 22.352) (end 48.514 22.352) (width 0.4) (layer "F.Cu") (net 9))
 (segment (start 43.852 20.23) (end 45.974 22.352) (width 0.4) (layer "F.Cu") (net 9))
 (segment (start 38.141 20.23) (end 39.751 20.23) (width 0.4) (layer "F.Cu") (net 9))
 (segment (start 37.821 20.55) (end 38.141 20.23) (width 0.4) (layer "F.Cu") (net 9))
 (segment (start 39.751 20.23) (end 43.852 20.23) (width 0.4) (layer "F.Cu") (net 9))
 (segment (start 37.9075 29.464) (end 38.354 29.9105) (width 0.25) (layer "F.Cu") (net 7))
 (segment (start 35.4 29.464) (end 37.9075 29.464) (width 0.25) (layer "F.Cu") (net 7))
 (segment (start 40.263 24.892) (end 37.821 22.45) (width 0.25) (layer "F.Cu") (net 8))
 (segment (start 48.514 24.892) (end 40.263 24.892) (width 0.25) (layer "F.Cu") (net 8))
 (segment (start 37.821 26.4525) (end 37.821 22.45) (width 0.25) (layer "F.Cu") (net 8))
 (segment (start 38.354 26.9855) (end 37.821 26.4525) (width 0.25) (layer "F.Cu") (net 8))
 (segment (start 37.084 28.448) (end 47.498 28.448) (width 0.25) (layer "F.Cu") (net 6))
 (segment (start 35.4625 26.8265) (end 37.084 28.448) (width 0.25) (layer "F.Cu") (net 6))
 (segment (start 35.331 25.6495) (end 35.4625 25.781) (width 0.25) (layer "F.Cu") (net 6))
 (segment (start 47.498 28.448) (end 48.514 27.432) (width 0.25) (layer "F.Cu") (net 6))
 (segment (start 35.4625 25.781) (end 35.4625 26.8265) (width 0.25) (layer "F.Cu") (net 6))
 (segment (start 35.331 22.45) (end 35.331 25.6495) (width 0.25) (layer "F.Cu") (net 6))
 (segment (start 30.226 24.4602) (end 27.94 22.1742) (width 0.25) (layer "F.Cu") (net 1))
 (segment (start 28.7782 21.336) (end 32.663 21.336) (width 0.35) (layer "F.Cu") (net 1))
 (segment (start 46.736 18.034) (end 34.036 18.034) (width 0.35) (layer "F.Cu") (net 1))
 (segment (start 48.514 19.812) (end 46.736 18.034) (width 0.35) (layer "F.Cu") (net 1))
 (segment (start 33.401 20.598) (end 35.283 20.598) (width 0.25) (layer "F.Cu") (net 1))
 (segment (start 30.226 27.436) (end 32.254 29.464) (width 0.25) (layer "F.Cu") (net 1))
 (segment (start 30.226 27.436) (end 30.226 24.4602) (width 0.25) (layer "F.Cu") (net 1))
 (segment (start 33.401 18.669) (end 33.401 20.598) (width 0.35) (layer "F.Cu") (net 1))
 (segment (start 27.94 22.1742) (end 28.7782 21.336) (width 0.35) (layer "F.Cu") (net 1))
 (segment (start 32.254 29.464) (end 32.6 29.464) (width 0.25) (layer "F.Cu") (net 1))
 (segment (start 32.663 21.336) (end 33.401 20.598) (width 0.35) (layer "F.Cu") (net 1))
 (segment (start 27.4142 22.7) (end 27.94 22.1742) (width 0.35) (layer "F.Cu") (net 1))
 (segment (start 22.86 22.7) (end 27.4142 22.7) (width 0.35) (layer "F.Cu") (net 1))
 (segment (start 34.036 18.034) (end 33.401 18.669) (width 0.35) (layer "F.Cu") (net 1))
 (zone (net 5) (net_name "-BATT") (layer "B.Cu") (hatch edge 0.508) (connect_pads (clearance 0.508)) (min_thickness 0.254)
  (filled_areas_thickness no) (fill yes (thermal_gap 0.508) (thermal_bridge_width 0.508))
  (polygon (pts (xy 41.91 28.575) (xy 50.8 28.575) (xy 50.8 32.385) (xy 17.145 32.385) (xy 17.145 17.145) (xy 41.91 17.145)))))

